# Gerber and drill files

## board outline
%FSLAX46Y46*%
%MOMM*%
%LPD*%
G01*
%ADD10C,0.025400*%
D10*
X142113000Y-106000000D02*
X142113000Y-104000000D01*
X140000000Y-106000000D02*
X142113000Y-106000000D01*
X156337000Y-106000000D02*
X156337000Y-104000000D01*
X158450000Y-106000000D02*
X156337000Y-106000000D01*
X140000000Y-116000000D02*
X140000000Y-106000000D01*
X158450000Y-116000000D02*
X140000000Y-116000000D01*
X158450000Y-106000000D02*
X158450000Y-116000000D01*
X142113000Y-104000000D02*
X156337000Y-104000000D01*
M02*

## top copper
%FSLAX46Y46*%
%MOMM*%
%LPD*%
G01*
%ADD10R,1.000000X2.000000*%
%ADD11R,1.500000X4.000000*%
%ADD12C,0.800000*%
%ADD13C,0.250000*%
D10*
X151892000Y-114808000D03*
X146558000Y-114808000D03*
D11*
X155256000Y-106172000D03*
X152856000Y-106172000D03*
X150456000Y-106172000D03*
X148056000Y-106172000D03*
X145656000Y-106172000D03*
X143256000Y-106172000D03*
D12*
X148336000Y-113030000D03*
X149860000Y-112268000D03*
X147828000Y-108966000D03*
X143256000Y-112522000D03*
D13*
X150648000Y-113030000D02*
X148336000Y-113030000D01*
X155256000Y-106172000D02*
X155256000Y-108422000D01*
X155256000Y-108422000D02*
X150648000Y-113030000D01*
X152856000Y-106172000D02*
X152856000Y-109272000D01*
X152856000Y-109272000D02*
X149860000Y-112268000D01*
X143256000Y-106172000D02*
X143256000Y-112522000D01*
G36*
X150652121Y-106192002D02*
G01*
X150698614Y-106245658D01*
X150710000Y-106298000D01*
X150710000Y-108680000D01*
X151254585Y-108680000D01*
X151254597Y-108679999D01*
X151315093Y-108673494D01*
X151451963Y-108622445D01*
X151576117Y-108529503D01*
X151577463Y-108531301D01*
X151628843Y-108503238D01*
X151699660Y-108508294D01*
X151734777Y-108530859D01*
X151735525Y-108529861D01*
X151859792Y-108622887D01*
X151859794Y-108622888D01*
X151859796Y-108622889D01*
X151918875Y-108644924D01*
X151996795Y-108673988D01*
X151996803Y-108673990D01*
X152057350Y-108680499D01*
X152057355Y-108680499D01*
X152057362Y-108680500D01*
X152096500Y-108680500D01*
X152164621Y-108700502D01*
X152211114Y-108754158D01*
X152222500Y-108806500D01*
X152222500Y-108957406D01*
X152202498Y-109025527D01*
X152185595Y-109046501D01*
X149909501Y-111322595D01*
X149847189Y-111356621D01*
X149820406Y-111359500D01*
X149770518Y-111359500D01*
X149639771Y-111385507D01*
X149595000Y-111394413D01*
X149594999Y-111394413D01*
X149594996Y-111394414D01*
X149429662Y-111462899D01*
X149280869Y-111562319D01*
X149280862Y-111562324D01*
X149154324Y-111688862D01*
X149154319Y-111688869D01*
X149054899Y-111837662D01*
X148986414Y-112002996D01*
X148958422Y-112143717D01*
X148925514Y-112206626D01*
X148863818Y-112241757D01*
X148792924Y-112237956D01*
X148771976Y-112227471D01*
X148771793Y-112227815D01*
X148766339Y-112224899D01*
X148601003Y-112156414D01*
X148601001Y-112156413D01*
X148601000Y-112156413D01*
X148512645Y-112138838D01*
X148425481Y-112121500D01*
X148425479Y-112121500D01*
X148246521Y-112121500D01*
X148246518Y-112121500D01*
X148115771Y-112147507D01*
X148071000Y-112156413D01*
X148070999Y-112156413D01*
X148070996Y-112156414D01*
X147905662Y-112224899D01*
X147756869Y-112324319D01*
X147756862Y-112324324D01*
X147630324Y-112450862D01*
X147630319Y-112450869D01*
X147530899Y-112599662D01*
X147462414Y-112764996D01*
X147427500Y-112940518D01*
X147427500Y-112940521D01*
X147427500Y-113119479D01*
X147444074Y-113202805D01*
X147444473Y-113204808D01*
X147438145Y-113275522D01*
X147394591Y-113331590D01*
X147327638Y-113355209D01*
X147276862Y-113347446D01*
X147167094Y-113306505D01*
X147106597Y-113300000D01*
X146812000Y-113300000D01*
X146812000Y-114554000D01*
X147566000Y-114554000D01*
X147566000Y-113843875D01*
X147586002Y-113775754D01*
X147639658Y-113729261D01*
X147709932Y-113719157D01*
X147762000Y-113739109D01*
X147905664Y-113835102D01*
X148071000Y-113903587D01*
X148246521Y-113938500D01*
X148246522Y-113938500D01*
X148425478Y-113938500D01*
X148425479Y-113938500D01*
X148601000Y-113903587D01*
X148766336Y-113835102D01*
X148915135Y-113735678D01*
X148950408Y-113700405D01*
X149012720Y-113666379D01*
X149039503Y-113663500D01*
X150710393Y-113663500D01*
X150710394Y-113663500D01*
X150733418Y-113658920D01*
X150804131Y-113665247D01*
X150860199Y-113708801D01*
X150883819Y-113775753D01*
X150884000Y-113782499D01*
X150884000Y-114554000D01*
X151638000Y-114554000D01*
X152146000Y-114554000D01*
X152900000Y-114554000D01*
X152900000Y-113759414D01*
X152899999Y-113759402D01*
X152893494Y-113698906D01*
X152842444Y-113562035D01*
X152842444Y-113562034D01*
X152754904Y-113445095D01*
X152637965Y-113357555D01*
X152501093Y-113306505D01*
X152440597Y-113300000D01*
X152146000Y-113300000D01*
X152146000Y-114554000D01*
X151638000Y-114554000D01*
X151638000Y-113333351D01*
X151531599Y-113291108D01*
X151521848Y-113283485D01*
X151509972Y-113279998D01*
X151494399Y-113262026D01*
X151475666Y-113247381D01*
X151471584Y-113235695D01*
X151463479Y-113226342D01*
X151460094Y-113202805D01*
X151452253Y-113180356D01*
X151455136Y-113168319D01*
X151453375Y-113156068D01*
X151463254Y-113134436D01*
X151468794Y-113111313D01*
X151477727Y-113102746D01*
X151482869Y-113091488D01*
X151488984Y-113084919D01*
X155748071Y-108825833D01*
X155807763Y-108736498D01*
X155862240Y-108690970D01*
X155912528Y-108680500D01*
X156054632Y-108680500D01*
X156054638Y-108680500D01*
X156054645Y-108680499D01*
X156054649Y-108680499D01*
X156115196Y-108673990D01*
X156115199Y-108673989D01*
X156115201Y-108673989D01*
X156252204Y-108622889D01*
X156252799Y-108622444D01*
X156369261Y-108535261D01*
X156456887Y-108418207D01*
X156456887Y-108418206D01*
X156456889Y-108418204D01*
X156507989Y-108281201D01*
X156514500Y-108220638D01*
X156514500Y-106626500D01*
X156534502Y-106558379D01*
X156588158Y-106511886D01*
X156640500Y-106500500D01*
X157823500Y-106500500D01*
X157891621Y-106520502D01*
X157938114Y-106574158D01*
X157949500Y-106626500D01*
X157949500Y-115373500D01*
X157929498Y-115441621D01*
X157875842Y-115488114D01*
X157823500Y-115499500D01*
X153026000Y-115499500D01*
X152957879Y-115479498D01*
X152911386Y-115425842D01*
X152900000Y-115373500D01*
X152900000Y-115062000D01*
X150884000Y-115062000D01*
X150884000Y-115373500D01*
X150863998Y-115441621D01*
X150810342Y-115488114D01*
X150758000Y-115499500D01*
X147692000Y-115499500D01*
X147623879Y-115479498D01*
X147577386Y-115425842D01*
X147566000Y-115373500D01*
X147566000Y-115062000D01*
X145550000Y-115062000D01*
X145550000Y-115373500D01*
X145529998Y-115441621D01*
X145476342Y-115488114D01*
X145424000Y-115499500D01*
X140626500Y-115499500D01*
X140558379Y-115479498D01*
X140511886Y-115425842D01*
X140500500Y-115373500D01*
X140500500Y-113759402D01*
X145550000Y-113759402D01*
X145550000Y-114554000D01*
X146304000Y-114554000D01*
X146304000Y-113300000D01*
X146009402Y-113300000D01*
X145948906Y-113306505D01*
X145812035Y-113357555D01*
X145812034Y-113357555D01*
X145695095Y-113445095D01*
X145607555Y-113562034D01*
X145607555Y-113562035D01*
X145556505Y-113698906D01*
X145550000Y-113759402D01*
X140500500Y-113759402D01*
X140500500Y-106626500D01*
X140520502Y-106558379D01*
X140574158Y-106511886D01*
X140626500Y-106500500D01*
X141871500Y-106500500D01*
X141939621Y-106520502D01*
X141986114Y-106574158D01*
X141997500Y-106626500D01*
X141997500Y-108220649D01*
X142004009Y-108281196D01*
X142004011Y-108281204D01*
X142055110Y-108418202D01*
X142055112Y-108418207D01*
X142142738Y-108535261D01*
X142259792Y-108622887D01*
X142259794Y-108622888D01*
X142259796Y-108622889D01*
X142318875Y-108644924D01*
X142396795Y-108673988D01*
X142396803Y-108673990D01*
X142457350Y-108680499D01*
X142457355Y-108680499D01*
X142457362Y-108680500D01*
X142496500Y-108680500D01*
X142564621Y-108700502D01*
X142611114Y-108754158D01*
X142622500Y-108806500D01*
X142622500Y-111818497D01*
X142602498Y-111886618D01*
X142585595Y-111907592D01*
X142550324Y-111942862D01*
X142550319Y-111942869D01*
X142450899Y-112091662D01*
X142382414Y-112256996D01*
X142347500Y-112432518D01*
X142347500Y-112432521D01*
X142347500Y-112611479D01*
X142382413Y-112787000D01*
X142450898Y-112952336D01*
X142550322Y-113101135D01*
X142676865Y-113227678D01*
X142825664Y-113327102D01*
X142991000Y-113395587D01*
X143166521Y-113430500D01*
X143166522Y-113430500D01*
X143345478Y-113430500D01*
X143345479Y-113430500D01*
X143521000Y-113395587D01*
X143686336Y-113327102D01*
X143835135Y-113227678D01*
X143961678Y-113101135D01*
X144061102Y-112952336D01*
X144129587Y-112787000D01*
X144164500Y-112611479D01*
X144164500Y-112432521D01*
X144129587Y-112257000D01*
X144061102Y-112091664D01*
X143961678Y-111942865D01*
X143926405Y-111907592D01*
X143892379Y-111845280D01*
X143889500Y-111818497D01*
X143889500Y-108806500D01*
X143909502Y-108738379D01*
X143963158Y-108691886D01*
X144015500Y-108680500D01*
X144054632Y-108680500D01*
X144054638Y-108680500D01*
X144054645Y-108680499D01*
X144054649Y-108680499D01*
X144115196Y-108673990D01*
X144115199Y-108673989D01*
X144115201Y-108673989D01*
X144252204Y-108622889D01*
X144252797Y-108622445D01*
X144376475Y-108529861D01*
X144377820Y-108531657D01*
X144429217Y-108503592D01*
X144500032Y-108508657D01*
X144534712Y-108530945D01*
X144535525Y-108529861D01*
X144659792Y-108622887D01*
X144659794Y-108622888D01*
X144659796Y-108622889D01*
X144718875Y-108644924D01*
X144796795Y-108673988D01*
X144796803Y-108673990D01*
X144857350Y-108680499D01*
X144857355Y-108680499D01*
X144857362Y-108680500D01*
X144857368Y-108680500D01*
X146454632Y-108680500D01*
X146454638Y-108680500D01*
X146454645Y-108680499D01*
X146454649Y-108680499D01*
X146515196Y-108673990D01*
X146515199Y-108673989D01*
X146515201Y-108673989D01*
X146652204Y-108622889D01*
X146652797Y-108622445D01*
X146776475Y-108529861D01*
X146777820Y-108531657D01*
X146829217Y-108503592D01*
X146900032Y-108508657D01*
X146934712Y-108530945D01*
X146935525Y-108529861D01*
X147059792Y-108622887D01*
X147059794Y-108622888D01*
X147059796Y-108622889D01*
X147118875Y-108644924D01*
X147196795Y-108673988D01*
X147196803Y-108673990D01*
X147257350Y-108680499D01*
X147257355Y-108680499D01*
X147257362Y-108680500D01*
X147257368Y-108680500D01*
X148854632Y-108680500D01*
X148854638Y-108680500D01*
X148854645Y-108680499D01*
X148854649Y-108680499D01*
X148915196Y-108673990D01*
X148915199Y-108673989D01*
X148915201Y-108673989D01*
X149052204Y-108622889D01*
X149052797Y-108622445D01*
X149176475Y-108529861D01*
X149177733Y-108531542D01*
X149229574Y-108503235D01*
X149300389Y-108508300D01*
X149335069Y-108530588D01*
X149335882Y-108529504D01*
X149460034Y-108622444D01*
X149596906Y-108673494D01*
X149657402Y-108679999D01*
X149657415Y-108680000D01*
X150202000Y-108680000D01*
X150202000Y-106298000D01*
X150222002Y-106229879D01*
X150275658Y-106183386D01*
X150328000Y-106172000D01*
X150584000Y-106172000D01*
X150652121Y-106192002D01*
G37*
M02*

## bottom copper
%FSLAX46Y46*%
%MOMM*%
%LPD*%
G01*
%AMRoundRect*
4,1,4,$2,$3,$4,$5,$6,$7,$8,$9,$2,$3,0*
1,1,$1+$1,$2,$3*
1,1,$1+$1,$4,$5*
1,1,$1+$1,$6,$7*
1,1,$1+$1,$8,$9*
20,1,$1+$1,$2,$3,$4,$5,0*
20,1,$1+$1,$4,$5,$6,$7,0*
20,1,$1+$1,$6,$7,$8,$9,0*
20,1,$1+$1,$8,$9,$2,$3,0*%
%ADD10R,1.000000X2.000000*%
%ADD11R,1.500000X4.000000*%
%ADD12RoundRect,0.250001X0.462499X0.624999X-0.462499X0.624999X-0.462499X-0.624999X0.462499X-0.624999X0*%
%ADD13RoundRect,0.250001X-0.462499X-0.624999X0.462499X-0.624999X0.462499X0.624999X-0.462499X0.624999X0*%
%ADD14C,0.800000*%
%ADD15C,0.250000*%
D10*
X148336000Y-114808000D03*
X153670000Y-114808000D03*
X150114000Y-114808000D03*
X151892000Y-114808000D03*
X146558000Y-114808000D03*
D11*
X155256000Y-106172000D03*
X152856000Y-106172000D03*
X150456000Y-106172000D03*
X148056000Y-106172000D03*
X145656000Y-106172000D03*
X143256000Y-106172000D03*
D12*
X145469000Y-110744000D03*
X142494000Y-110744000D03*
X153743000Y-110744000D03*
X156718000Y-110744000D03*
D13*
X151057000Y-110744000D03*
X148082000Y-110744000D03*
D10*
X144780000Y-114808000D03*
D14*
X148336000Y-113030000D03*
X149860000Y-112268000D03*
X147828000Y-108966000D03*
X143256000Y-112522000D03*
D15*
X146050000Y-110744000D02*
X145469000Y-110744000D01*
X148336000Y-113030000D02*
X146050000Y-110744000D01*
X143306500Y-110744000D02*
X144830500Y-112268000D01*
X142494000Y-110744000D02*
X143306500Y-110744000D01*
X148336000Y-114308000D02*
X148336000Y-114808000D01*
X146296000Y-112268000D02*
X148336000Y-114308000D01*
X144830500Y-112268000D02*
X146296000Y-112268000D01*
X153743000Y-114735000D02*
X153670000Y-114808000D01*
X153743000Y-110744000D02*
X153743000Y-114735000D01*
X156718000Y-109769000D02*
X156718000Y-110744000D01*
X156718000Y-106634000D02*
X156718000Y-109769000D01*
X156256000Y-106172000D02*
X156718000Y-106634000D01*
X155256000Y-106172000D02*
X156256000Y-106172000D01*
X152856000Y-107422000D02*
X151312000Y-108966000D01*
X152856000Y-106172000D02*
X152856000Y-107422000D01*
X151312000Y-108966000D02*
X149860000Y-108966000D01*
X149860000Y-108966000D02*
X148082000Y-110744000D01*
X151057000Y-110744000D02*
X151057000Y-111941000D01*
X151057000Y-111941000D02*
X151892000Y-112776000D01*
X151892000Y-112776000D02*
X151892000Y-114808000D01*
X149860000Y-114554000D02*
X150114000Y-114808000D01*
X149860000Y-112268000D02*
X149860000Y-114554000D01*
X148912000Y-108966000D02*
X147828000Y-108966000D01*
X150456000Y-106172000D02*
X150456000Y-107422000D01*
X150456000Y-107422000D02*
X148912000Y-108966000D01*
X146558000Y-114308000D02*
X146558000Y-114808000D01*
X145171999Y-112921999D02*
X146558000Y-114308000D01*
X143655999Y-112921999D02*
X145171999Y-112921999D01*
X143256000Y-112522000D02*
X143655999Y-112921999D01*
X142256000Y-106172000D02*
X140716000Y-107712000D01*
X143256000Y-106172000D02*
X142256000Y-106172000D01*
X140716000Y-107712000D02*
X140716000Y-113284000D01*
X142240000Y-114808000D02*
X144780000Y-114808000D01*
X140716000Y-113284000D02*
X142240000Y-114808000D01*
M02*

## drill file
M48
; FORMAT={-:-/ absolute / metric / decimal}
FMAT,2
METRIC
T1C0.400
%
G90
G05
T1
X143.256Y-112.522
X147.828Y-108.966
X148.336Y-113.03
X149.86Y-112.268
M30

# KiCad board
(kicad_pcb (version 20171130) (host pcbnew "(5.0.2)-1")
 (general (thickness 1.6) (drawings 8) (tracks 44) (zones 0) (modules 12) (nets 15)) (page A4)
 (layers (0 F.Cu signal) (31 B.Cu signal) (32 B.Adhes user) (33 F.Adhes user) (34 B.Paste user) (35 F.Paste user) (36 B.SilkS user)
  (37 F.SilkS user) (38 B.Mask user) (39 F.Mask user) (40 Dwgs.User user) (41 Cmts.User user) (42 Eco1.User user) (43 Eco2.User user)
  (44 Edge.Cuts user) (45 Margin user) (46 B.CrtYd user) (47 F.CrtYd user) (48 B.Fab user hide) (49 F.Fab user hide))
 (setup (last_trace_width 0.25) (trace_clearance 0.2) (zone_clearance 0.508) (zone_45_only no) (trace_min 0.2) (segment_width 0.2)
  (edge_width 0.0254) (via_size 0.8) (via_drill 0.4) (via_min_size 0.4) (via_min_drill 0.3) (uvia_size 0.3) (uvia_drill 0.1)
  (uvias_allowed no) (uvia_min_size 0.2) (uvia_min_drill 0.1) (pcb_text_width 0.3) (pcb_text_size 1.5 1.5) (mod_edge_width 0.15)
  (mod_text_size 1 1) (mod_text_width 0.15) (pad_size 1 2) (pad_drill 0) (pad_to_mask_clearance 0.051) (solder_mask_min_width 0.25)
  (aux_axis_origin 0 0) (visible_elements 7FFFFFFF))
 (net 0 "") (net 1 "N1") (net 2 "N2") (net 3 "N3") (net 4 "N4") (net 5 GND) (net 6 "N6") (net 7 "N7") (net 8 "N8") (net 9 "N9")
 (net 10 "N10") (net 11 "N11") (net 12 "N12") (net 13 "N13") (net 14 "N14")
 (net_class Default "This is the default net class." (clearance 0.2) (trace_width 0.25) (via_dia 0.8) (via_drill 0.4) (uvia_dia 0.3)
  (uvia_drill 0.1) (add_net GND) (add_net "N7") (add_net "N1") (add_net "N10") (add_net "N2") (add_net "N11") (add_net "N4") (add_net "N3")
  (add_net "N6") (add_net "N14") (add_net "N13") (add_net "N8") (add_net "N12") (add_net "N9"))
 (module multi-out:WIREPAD (layer B.Cu) (at 148.336 114.808)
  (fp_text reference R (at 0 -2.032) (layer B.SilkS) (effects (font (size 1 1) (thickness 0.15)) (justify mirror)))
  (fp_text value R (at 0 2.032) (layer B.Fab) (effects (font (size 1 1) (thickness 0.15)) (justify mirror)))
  (pad 1 connect rect (at 0 0) (size 1 2) (layers B.Cu B.Mask) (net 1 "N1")))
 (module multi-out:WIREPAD (layer B.Cu) (at 153.67 114.808)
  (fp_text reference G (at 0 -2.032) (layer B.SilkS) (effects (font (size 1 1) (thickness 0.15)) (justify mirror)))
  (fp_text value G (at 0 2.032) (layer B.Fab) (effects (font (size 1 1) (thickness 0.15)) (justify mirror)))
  (pad 1 connect rect (at 0 0) (size 1 2) (layers B.Cu B.Mask) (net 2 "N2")))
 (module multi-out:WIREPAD (layer B.Cu) (at 150.114 114.808)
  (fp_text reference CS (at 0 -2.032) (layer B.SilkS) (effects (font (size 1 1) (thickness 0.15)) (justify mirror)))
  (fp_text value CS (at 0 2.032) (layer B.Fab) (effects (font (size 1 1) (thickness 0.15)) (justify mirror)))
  (pad 1 connect rect (at 0 0) (size 1 2) (layers B.Cu B.Mask) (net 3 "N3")))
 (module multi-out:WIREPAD (layer B.Cu) (at 151.892 114.808)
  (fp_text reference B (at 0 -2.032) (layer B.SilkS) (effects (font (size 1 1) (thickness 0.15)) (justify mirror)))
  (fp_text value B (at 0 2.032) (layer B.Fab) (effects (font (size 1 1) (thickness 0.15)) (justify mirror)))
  (pad 1 connect rect (at 0 0) (size 1 2) (layers B.Cu B.Mask) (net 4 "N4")))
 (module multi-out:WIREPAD (layer F.Cu) (at 151.892 114.808)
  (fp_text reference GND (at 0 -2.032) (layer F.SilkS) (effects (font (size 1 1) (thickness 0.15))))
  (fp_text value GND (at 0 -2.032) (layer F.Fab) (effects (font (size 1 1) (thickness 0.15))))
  (pad 1 connect rect (at 0 0) (size 1 2) (layers F.Cu F.Mask) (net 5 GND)))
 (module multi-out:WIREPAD (layer F.Cu) (at 146.558 114.808)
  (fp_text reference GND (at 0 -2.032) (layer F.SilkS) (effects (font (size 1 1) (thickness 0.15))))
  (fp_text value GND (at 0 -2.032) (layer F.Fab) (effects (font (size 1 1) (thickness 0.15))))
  (pad 1 connect rect (at 0 0) (size 1 2) (layers F.Cu F.Mask) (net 5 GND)))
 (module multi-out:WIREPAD (layer B.Cu) (at 146.558 114.808)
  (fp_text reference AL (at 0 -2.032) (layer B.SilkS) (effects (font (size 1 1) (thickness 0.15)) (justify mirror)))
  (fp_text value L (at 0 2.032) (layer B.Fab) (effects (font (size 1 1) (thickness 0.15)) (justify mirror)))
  (pad 1 connect rect (at 0 0) (size 1 2) (layers B.Cu B.Mask) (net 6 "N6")))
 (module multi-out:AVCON (layer F.Cu) (at 149.16 106.172)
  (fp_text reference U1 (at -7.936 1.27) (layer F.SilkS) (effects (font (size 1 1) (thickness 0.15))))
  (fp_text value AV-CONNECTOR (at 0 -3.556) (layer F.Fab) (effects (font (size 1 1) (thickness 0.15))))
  (pad 1 connect rect (at 6.096 0) (size 1.5 4) (layers F.Cu F.Mask) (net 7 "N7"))
  (pad 3 connect rect (at 3.696 0) (size 1.5 4) (layers F.Cu F.Mask) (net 3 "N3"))
  (pad 5 connect rect (at 1.296 0) (size 1.5 4) (layers F.Cu F.Mask) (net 5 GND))
  (pad 7 connect rect (at -1.104 0) (size 1.5 4) (layers F.Cu F.Mask) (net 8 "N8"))
  (pad 9 connect rect (at -3.504 0) (size 1.5 4) (layers F.Cu F.Mask) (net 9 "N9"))
  (pad 11 connect rect (at -5.904 0) (size 1.5 4) (layers F.Cu F.Mask) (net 6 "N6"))
  (pad 2 connect rect (at 6.096 0) (size 1.5 4) (layers B.Cu B.Mask) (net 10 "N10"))
  (pad 4 connect rect (at 3.696 0) (size 1.5 4) (layers B.Cu B.Mask) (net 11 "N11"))
  (pad 6 connect rect (at 1.296 0) (size 1.5 4) (layers B.Cu B.Mask) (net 5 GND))
  (pad 8 connect rect (at -1.104 0) (size 1.5 4) (layers B.Cu B.Mask) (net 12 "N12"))
  (pad 10 connect rect (at -3.504 0) (size 1.5 4) (layers B.Cu B.Mask) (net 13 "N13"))
  (pad 12 connect rect (at -5.904 0) (size 1.5 4) (layers B.Cu B.Mask) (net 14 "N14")))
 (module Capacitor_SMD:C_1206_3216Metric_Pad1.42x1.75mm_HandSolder (layer B.Cu) (at 143.9815 110.744 180)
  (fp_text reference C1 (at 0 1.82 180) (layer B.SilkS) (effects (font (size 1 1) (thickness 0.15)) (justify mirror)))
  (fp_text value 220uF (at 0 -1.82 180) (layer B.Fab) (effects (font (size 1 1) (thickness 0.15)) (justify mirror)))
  (pad 1 smd roundrect (at -1.4875 0 180) (size 1.425 1.75) (layers B.Cu B.Paste B.Mask) (roundrect_rratio 0.175439) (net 7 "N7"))
  (pad 2 smd roundrect (at 1.4875 0 180) (size 1.425 1.75) (layers B.Cu B.Paste B.Mask) (roundrect_rratio 0.175439) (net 1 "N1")))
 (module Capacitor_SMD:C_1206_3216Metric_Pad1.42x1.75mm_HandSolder (layer B.Cu) (at 155.2305 110.744 180)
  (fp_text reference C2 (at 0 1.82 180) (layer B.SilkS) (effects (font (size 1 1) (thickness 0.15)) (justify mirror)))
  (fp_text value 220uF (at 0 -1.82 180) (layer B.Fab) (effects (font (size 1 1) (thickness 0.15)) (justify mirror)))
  (pad 2 smd roundrect (at 1.4875 0 180) (size 1.425 1.75) (layers B.Cu B.Paste B.Mask) (roundrect_rratio 0.175439) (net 2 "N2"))
  (pad 1 smd roundrect (at -1.4875 0 180) (size 1.425 1.75) (layers B.Cu B.Paste B.Mask) (roundrect_rratio 0.175439) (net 10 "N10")))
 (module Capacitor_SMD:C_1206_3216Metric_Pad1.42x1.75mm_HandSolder (layer B.Cu) (at 149.5695 110.744)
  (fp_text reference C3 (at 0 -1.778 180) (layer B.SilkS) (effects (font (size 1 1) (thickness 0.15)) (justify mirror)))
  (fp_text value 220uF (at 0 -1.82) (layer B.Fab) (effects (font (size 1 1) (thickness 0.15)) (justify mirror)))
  (pad 2 smd roundrect (at 1.4875 0) (size 1.425 1.75) (layers B.Cu B.Paste B.Mask) (roundrect_rratio 0.175439) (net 4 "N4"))
  (pad 1 smd roundrect (at -1.4875 0) (size 1.425 1.75) (layers B.Cu B.Paste B.Mask) (roundrect_rratio 0.175439) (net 11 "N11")))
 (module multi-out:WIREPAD (layer B.Cu) (at 144.78 114.808)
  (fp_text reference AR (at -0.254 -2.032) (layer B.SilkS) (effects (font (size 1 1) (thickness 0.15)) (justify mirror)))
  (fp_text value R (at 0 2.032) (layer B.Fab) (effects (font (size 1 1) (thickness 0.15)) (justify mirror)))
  (pad 1 connect rect (at 0 0) (size 1 2) (layers B.Cu B.Mask) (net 14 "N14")))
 (gr_line (start 142.113 106) (end 142.113 104) (layer Edge.Cuts) (width 0.0254))
 (gr_line (start 140 106) (end 142.113 106) (layer Edge.Cuts) (width 0.0254))
 (gr_line (start 156.337 106) (end 156.337 104) (layer Edge.Cuts) (width 0.0254))
 (gr_line (start 158.45 106) (end 156.337 106) (layer Edge.Cuts) (width 0.0254))
 (gr_line (start 140 116) (end 140 106) (layer Edge.Cuts) (width 0.0254))
 (gr_line (start 158.45 116) (end 140 116) (layer Edge.Cuts) (width 0.0254))
 (gr_line (start 158.45 106) (end 158.45 116) (layer Edge.Cuts) (width 0.0254))
 (gr_line (start 142.113 104) (end 156.337 104) (layer Edge.Cuts) (width 0.0254))
 (via (at 148.336 113.03) (size 0.8) (drill 0.4) (layers F.Cu B.Cu) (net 7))
 (segment (start 150.648 113.03) (end 148.336 113.03) (width 0.25) (layer F.Cu) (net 7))
 (segment (start 155.256 106.172) (end 155.256 108.422) (width 0.25) (layer F.Cu) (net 7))
 (segment (start 155.256 108.422) (end 150.648 113.03) (width 0.25) (layer F.Cu) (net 7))
 (segment (start 146.05 110.744) (end 145.469 110.744) (width 0.25) (layer B.Cu) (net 7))
 (segment (start 148.336 113.03) (end 146.05 110.744) (width 0.25) (layer B.Cu) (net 7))
 (segment (start 143.3065 110.744) (end 144.8305 112.268) (width 0.25) (layer B.Cu) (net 1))
 (segment (start 142.494 110.744) (end 143.3065 110.744) (width 0.25) (layer B.Cu) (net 1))
 (segment (start 148.336 114.308) (end 148.336 114.808) (width 0.25) (layer B.Cu) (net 1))
 (segment (start 146.296 112.268) (end 148.336 114.308) (width 0.25) (layer B.Cu) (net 1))
 (segment (start 144.8305 112.268) (end 146.296 112.268) (width 0.25) (layer B.Cu) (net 1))
 (segment (start 153.743 114.735) (end 153.67 114.808) (width 0.25) (layer B.Cu) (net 2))
 (segment (start 153.743 110.744) (end 153.743 114.735) (width 0.25) (layer B.Cu) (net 2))
 (segment (start 156.718 109.769) (end 156.718 110.744) (width 0.25) (layer B.Cu) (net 10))
 (segment (start 156.718 106.634) (end 156.718 109.769) (width 0.25) (layer B.Cu) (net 10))
 (segment (start 156.256 106.172) (end 156.718 106.634) (width 0.25) (layer B.Cu) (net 10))
 (segment (start 155.256 106.172) (end 156.256 106.172) (width 0.25) (layer B.Cu) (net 10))
 (segment (start 152.856 107.422) (end 151.312 108.966) (width 0.25) (layer B.Cu) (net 11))
 (segment (start 152.856 106.172) (end 152.856 107.422) (width 0.25) (layer B.Cu) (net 11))
 (segment (start 151.312 108.966) (end 149.86 108.966) (width 0.25) (layer B.Cu) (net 11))
 (segment (start 149.86 108.966) (end 148.082 110.744) (width 0.25) (layer B.Cu) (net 11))
 (segment (start 151.057 110.744) (end 151.057 111.941) (width 0.25) (layer B.Cu) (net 4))
 (segment (start 151.057 111.941) (end 151.892 112.776) (width 0.25) (layer B.Cu) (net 4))
 (segment (start 151.892 112.776) (end 151.892 114.808) (width 0.25) (layer B.Cu) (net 4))
 (via (at 149.86 112.268) (size 0.8) (drill 0.4) (layers F.Cu B.Cu) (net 3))
 (segment (start 152.856 106.172) (end 152.856 109.272) (width 0.25) (layer F.Cu) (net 3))
 (segment (start 152.856 109.272) (end 149.86 112.268) (width 0.25) (layer F.Cu) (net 3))
 (segment (start 149.86 114.554) (end 150.114 114.808) (width 0.25) (layer B.Cu) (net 3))
 (segment (start 149.86 112.268) (end 149.86 114.554) (width 0.25) (layer B.Cu) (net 3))
 (via (at 147.828 108.966) (size 0.8) (drill 0.4) (layers F.Cu B.Cu) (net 5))
 (segment (start 148.912 108.966) (end 147.828 108.966) (width 0.25) (layer B.Cu) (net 5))
 (segment (start 150.456 106.172) (end 150.456 107.422) (width 0.25) (layer B.Cu) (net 5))
 (segment (start 150.456 107.422) (end 148.912 108.966) (width 0.25) (layer B.Cu) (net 5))
 (via (at 143.256 112.522) (size 0.8) (drill 0.4) (layers F.Cu B.Cu) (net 6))
 (segment (start 143.256 106.172) (end 143.256 112.522) (width 0.25) (layer F.Cu) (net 6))
 (segment (start 146.558 114.308) (end 146.558 114.808) (width 0.25) (layer B.Cu) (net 6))
 (segment (start 145.171999 112.921999) (end 146.558 114.308) (width 0.25) (layer B.Cu) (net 6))
 (segment (start 143.655999 112.921999) (end 145.171999 112.921999) (width 0.25) (layer B.Cu) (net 6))
 (segment (start 143.256 112.522) (end 143.655999 112.921999) (width 0.25) (layer B.Cu) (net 6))
 (segment (start 142.256 106.172) (end 140.716 107.712) (width 0.25) (layer B.Cu) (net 14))
 (segment (start 143.256 106.172) (end 142.256 106.172) (width 0.25) (layer B.Cu) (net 14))
 (segment (start 140.716 107.712) (end 140.716 113.284) (width 0.25) (layer B.Cu) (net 14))
 (segment (start 142.24 114.808) (end 144.78 114.808) (width 0.25) (layer B.Cu) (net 14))
 (segment (start 140.716 113.284) (end 142.24 114.808) (width 0.25) (layer B.Cu) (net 14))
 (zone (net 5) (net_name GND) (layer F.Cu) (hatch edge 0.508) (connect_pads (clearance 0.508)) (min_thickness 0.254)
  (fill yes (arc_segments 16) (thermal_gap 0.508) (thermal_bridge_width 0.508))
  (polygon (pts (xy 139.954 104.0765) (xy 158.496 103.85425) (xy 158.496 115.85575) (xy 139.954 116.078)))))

